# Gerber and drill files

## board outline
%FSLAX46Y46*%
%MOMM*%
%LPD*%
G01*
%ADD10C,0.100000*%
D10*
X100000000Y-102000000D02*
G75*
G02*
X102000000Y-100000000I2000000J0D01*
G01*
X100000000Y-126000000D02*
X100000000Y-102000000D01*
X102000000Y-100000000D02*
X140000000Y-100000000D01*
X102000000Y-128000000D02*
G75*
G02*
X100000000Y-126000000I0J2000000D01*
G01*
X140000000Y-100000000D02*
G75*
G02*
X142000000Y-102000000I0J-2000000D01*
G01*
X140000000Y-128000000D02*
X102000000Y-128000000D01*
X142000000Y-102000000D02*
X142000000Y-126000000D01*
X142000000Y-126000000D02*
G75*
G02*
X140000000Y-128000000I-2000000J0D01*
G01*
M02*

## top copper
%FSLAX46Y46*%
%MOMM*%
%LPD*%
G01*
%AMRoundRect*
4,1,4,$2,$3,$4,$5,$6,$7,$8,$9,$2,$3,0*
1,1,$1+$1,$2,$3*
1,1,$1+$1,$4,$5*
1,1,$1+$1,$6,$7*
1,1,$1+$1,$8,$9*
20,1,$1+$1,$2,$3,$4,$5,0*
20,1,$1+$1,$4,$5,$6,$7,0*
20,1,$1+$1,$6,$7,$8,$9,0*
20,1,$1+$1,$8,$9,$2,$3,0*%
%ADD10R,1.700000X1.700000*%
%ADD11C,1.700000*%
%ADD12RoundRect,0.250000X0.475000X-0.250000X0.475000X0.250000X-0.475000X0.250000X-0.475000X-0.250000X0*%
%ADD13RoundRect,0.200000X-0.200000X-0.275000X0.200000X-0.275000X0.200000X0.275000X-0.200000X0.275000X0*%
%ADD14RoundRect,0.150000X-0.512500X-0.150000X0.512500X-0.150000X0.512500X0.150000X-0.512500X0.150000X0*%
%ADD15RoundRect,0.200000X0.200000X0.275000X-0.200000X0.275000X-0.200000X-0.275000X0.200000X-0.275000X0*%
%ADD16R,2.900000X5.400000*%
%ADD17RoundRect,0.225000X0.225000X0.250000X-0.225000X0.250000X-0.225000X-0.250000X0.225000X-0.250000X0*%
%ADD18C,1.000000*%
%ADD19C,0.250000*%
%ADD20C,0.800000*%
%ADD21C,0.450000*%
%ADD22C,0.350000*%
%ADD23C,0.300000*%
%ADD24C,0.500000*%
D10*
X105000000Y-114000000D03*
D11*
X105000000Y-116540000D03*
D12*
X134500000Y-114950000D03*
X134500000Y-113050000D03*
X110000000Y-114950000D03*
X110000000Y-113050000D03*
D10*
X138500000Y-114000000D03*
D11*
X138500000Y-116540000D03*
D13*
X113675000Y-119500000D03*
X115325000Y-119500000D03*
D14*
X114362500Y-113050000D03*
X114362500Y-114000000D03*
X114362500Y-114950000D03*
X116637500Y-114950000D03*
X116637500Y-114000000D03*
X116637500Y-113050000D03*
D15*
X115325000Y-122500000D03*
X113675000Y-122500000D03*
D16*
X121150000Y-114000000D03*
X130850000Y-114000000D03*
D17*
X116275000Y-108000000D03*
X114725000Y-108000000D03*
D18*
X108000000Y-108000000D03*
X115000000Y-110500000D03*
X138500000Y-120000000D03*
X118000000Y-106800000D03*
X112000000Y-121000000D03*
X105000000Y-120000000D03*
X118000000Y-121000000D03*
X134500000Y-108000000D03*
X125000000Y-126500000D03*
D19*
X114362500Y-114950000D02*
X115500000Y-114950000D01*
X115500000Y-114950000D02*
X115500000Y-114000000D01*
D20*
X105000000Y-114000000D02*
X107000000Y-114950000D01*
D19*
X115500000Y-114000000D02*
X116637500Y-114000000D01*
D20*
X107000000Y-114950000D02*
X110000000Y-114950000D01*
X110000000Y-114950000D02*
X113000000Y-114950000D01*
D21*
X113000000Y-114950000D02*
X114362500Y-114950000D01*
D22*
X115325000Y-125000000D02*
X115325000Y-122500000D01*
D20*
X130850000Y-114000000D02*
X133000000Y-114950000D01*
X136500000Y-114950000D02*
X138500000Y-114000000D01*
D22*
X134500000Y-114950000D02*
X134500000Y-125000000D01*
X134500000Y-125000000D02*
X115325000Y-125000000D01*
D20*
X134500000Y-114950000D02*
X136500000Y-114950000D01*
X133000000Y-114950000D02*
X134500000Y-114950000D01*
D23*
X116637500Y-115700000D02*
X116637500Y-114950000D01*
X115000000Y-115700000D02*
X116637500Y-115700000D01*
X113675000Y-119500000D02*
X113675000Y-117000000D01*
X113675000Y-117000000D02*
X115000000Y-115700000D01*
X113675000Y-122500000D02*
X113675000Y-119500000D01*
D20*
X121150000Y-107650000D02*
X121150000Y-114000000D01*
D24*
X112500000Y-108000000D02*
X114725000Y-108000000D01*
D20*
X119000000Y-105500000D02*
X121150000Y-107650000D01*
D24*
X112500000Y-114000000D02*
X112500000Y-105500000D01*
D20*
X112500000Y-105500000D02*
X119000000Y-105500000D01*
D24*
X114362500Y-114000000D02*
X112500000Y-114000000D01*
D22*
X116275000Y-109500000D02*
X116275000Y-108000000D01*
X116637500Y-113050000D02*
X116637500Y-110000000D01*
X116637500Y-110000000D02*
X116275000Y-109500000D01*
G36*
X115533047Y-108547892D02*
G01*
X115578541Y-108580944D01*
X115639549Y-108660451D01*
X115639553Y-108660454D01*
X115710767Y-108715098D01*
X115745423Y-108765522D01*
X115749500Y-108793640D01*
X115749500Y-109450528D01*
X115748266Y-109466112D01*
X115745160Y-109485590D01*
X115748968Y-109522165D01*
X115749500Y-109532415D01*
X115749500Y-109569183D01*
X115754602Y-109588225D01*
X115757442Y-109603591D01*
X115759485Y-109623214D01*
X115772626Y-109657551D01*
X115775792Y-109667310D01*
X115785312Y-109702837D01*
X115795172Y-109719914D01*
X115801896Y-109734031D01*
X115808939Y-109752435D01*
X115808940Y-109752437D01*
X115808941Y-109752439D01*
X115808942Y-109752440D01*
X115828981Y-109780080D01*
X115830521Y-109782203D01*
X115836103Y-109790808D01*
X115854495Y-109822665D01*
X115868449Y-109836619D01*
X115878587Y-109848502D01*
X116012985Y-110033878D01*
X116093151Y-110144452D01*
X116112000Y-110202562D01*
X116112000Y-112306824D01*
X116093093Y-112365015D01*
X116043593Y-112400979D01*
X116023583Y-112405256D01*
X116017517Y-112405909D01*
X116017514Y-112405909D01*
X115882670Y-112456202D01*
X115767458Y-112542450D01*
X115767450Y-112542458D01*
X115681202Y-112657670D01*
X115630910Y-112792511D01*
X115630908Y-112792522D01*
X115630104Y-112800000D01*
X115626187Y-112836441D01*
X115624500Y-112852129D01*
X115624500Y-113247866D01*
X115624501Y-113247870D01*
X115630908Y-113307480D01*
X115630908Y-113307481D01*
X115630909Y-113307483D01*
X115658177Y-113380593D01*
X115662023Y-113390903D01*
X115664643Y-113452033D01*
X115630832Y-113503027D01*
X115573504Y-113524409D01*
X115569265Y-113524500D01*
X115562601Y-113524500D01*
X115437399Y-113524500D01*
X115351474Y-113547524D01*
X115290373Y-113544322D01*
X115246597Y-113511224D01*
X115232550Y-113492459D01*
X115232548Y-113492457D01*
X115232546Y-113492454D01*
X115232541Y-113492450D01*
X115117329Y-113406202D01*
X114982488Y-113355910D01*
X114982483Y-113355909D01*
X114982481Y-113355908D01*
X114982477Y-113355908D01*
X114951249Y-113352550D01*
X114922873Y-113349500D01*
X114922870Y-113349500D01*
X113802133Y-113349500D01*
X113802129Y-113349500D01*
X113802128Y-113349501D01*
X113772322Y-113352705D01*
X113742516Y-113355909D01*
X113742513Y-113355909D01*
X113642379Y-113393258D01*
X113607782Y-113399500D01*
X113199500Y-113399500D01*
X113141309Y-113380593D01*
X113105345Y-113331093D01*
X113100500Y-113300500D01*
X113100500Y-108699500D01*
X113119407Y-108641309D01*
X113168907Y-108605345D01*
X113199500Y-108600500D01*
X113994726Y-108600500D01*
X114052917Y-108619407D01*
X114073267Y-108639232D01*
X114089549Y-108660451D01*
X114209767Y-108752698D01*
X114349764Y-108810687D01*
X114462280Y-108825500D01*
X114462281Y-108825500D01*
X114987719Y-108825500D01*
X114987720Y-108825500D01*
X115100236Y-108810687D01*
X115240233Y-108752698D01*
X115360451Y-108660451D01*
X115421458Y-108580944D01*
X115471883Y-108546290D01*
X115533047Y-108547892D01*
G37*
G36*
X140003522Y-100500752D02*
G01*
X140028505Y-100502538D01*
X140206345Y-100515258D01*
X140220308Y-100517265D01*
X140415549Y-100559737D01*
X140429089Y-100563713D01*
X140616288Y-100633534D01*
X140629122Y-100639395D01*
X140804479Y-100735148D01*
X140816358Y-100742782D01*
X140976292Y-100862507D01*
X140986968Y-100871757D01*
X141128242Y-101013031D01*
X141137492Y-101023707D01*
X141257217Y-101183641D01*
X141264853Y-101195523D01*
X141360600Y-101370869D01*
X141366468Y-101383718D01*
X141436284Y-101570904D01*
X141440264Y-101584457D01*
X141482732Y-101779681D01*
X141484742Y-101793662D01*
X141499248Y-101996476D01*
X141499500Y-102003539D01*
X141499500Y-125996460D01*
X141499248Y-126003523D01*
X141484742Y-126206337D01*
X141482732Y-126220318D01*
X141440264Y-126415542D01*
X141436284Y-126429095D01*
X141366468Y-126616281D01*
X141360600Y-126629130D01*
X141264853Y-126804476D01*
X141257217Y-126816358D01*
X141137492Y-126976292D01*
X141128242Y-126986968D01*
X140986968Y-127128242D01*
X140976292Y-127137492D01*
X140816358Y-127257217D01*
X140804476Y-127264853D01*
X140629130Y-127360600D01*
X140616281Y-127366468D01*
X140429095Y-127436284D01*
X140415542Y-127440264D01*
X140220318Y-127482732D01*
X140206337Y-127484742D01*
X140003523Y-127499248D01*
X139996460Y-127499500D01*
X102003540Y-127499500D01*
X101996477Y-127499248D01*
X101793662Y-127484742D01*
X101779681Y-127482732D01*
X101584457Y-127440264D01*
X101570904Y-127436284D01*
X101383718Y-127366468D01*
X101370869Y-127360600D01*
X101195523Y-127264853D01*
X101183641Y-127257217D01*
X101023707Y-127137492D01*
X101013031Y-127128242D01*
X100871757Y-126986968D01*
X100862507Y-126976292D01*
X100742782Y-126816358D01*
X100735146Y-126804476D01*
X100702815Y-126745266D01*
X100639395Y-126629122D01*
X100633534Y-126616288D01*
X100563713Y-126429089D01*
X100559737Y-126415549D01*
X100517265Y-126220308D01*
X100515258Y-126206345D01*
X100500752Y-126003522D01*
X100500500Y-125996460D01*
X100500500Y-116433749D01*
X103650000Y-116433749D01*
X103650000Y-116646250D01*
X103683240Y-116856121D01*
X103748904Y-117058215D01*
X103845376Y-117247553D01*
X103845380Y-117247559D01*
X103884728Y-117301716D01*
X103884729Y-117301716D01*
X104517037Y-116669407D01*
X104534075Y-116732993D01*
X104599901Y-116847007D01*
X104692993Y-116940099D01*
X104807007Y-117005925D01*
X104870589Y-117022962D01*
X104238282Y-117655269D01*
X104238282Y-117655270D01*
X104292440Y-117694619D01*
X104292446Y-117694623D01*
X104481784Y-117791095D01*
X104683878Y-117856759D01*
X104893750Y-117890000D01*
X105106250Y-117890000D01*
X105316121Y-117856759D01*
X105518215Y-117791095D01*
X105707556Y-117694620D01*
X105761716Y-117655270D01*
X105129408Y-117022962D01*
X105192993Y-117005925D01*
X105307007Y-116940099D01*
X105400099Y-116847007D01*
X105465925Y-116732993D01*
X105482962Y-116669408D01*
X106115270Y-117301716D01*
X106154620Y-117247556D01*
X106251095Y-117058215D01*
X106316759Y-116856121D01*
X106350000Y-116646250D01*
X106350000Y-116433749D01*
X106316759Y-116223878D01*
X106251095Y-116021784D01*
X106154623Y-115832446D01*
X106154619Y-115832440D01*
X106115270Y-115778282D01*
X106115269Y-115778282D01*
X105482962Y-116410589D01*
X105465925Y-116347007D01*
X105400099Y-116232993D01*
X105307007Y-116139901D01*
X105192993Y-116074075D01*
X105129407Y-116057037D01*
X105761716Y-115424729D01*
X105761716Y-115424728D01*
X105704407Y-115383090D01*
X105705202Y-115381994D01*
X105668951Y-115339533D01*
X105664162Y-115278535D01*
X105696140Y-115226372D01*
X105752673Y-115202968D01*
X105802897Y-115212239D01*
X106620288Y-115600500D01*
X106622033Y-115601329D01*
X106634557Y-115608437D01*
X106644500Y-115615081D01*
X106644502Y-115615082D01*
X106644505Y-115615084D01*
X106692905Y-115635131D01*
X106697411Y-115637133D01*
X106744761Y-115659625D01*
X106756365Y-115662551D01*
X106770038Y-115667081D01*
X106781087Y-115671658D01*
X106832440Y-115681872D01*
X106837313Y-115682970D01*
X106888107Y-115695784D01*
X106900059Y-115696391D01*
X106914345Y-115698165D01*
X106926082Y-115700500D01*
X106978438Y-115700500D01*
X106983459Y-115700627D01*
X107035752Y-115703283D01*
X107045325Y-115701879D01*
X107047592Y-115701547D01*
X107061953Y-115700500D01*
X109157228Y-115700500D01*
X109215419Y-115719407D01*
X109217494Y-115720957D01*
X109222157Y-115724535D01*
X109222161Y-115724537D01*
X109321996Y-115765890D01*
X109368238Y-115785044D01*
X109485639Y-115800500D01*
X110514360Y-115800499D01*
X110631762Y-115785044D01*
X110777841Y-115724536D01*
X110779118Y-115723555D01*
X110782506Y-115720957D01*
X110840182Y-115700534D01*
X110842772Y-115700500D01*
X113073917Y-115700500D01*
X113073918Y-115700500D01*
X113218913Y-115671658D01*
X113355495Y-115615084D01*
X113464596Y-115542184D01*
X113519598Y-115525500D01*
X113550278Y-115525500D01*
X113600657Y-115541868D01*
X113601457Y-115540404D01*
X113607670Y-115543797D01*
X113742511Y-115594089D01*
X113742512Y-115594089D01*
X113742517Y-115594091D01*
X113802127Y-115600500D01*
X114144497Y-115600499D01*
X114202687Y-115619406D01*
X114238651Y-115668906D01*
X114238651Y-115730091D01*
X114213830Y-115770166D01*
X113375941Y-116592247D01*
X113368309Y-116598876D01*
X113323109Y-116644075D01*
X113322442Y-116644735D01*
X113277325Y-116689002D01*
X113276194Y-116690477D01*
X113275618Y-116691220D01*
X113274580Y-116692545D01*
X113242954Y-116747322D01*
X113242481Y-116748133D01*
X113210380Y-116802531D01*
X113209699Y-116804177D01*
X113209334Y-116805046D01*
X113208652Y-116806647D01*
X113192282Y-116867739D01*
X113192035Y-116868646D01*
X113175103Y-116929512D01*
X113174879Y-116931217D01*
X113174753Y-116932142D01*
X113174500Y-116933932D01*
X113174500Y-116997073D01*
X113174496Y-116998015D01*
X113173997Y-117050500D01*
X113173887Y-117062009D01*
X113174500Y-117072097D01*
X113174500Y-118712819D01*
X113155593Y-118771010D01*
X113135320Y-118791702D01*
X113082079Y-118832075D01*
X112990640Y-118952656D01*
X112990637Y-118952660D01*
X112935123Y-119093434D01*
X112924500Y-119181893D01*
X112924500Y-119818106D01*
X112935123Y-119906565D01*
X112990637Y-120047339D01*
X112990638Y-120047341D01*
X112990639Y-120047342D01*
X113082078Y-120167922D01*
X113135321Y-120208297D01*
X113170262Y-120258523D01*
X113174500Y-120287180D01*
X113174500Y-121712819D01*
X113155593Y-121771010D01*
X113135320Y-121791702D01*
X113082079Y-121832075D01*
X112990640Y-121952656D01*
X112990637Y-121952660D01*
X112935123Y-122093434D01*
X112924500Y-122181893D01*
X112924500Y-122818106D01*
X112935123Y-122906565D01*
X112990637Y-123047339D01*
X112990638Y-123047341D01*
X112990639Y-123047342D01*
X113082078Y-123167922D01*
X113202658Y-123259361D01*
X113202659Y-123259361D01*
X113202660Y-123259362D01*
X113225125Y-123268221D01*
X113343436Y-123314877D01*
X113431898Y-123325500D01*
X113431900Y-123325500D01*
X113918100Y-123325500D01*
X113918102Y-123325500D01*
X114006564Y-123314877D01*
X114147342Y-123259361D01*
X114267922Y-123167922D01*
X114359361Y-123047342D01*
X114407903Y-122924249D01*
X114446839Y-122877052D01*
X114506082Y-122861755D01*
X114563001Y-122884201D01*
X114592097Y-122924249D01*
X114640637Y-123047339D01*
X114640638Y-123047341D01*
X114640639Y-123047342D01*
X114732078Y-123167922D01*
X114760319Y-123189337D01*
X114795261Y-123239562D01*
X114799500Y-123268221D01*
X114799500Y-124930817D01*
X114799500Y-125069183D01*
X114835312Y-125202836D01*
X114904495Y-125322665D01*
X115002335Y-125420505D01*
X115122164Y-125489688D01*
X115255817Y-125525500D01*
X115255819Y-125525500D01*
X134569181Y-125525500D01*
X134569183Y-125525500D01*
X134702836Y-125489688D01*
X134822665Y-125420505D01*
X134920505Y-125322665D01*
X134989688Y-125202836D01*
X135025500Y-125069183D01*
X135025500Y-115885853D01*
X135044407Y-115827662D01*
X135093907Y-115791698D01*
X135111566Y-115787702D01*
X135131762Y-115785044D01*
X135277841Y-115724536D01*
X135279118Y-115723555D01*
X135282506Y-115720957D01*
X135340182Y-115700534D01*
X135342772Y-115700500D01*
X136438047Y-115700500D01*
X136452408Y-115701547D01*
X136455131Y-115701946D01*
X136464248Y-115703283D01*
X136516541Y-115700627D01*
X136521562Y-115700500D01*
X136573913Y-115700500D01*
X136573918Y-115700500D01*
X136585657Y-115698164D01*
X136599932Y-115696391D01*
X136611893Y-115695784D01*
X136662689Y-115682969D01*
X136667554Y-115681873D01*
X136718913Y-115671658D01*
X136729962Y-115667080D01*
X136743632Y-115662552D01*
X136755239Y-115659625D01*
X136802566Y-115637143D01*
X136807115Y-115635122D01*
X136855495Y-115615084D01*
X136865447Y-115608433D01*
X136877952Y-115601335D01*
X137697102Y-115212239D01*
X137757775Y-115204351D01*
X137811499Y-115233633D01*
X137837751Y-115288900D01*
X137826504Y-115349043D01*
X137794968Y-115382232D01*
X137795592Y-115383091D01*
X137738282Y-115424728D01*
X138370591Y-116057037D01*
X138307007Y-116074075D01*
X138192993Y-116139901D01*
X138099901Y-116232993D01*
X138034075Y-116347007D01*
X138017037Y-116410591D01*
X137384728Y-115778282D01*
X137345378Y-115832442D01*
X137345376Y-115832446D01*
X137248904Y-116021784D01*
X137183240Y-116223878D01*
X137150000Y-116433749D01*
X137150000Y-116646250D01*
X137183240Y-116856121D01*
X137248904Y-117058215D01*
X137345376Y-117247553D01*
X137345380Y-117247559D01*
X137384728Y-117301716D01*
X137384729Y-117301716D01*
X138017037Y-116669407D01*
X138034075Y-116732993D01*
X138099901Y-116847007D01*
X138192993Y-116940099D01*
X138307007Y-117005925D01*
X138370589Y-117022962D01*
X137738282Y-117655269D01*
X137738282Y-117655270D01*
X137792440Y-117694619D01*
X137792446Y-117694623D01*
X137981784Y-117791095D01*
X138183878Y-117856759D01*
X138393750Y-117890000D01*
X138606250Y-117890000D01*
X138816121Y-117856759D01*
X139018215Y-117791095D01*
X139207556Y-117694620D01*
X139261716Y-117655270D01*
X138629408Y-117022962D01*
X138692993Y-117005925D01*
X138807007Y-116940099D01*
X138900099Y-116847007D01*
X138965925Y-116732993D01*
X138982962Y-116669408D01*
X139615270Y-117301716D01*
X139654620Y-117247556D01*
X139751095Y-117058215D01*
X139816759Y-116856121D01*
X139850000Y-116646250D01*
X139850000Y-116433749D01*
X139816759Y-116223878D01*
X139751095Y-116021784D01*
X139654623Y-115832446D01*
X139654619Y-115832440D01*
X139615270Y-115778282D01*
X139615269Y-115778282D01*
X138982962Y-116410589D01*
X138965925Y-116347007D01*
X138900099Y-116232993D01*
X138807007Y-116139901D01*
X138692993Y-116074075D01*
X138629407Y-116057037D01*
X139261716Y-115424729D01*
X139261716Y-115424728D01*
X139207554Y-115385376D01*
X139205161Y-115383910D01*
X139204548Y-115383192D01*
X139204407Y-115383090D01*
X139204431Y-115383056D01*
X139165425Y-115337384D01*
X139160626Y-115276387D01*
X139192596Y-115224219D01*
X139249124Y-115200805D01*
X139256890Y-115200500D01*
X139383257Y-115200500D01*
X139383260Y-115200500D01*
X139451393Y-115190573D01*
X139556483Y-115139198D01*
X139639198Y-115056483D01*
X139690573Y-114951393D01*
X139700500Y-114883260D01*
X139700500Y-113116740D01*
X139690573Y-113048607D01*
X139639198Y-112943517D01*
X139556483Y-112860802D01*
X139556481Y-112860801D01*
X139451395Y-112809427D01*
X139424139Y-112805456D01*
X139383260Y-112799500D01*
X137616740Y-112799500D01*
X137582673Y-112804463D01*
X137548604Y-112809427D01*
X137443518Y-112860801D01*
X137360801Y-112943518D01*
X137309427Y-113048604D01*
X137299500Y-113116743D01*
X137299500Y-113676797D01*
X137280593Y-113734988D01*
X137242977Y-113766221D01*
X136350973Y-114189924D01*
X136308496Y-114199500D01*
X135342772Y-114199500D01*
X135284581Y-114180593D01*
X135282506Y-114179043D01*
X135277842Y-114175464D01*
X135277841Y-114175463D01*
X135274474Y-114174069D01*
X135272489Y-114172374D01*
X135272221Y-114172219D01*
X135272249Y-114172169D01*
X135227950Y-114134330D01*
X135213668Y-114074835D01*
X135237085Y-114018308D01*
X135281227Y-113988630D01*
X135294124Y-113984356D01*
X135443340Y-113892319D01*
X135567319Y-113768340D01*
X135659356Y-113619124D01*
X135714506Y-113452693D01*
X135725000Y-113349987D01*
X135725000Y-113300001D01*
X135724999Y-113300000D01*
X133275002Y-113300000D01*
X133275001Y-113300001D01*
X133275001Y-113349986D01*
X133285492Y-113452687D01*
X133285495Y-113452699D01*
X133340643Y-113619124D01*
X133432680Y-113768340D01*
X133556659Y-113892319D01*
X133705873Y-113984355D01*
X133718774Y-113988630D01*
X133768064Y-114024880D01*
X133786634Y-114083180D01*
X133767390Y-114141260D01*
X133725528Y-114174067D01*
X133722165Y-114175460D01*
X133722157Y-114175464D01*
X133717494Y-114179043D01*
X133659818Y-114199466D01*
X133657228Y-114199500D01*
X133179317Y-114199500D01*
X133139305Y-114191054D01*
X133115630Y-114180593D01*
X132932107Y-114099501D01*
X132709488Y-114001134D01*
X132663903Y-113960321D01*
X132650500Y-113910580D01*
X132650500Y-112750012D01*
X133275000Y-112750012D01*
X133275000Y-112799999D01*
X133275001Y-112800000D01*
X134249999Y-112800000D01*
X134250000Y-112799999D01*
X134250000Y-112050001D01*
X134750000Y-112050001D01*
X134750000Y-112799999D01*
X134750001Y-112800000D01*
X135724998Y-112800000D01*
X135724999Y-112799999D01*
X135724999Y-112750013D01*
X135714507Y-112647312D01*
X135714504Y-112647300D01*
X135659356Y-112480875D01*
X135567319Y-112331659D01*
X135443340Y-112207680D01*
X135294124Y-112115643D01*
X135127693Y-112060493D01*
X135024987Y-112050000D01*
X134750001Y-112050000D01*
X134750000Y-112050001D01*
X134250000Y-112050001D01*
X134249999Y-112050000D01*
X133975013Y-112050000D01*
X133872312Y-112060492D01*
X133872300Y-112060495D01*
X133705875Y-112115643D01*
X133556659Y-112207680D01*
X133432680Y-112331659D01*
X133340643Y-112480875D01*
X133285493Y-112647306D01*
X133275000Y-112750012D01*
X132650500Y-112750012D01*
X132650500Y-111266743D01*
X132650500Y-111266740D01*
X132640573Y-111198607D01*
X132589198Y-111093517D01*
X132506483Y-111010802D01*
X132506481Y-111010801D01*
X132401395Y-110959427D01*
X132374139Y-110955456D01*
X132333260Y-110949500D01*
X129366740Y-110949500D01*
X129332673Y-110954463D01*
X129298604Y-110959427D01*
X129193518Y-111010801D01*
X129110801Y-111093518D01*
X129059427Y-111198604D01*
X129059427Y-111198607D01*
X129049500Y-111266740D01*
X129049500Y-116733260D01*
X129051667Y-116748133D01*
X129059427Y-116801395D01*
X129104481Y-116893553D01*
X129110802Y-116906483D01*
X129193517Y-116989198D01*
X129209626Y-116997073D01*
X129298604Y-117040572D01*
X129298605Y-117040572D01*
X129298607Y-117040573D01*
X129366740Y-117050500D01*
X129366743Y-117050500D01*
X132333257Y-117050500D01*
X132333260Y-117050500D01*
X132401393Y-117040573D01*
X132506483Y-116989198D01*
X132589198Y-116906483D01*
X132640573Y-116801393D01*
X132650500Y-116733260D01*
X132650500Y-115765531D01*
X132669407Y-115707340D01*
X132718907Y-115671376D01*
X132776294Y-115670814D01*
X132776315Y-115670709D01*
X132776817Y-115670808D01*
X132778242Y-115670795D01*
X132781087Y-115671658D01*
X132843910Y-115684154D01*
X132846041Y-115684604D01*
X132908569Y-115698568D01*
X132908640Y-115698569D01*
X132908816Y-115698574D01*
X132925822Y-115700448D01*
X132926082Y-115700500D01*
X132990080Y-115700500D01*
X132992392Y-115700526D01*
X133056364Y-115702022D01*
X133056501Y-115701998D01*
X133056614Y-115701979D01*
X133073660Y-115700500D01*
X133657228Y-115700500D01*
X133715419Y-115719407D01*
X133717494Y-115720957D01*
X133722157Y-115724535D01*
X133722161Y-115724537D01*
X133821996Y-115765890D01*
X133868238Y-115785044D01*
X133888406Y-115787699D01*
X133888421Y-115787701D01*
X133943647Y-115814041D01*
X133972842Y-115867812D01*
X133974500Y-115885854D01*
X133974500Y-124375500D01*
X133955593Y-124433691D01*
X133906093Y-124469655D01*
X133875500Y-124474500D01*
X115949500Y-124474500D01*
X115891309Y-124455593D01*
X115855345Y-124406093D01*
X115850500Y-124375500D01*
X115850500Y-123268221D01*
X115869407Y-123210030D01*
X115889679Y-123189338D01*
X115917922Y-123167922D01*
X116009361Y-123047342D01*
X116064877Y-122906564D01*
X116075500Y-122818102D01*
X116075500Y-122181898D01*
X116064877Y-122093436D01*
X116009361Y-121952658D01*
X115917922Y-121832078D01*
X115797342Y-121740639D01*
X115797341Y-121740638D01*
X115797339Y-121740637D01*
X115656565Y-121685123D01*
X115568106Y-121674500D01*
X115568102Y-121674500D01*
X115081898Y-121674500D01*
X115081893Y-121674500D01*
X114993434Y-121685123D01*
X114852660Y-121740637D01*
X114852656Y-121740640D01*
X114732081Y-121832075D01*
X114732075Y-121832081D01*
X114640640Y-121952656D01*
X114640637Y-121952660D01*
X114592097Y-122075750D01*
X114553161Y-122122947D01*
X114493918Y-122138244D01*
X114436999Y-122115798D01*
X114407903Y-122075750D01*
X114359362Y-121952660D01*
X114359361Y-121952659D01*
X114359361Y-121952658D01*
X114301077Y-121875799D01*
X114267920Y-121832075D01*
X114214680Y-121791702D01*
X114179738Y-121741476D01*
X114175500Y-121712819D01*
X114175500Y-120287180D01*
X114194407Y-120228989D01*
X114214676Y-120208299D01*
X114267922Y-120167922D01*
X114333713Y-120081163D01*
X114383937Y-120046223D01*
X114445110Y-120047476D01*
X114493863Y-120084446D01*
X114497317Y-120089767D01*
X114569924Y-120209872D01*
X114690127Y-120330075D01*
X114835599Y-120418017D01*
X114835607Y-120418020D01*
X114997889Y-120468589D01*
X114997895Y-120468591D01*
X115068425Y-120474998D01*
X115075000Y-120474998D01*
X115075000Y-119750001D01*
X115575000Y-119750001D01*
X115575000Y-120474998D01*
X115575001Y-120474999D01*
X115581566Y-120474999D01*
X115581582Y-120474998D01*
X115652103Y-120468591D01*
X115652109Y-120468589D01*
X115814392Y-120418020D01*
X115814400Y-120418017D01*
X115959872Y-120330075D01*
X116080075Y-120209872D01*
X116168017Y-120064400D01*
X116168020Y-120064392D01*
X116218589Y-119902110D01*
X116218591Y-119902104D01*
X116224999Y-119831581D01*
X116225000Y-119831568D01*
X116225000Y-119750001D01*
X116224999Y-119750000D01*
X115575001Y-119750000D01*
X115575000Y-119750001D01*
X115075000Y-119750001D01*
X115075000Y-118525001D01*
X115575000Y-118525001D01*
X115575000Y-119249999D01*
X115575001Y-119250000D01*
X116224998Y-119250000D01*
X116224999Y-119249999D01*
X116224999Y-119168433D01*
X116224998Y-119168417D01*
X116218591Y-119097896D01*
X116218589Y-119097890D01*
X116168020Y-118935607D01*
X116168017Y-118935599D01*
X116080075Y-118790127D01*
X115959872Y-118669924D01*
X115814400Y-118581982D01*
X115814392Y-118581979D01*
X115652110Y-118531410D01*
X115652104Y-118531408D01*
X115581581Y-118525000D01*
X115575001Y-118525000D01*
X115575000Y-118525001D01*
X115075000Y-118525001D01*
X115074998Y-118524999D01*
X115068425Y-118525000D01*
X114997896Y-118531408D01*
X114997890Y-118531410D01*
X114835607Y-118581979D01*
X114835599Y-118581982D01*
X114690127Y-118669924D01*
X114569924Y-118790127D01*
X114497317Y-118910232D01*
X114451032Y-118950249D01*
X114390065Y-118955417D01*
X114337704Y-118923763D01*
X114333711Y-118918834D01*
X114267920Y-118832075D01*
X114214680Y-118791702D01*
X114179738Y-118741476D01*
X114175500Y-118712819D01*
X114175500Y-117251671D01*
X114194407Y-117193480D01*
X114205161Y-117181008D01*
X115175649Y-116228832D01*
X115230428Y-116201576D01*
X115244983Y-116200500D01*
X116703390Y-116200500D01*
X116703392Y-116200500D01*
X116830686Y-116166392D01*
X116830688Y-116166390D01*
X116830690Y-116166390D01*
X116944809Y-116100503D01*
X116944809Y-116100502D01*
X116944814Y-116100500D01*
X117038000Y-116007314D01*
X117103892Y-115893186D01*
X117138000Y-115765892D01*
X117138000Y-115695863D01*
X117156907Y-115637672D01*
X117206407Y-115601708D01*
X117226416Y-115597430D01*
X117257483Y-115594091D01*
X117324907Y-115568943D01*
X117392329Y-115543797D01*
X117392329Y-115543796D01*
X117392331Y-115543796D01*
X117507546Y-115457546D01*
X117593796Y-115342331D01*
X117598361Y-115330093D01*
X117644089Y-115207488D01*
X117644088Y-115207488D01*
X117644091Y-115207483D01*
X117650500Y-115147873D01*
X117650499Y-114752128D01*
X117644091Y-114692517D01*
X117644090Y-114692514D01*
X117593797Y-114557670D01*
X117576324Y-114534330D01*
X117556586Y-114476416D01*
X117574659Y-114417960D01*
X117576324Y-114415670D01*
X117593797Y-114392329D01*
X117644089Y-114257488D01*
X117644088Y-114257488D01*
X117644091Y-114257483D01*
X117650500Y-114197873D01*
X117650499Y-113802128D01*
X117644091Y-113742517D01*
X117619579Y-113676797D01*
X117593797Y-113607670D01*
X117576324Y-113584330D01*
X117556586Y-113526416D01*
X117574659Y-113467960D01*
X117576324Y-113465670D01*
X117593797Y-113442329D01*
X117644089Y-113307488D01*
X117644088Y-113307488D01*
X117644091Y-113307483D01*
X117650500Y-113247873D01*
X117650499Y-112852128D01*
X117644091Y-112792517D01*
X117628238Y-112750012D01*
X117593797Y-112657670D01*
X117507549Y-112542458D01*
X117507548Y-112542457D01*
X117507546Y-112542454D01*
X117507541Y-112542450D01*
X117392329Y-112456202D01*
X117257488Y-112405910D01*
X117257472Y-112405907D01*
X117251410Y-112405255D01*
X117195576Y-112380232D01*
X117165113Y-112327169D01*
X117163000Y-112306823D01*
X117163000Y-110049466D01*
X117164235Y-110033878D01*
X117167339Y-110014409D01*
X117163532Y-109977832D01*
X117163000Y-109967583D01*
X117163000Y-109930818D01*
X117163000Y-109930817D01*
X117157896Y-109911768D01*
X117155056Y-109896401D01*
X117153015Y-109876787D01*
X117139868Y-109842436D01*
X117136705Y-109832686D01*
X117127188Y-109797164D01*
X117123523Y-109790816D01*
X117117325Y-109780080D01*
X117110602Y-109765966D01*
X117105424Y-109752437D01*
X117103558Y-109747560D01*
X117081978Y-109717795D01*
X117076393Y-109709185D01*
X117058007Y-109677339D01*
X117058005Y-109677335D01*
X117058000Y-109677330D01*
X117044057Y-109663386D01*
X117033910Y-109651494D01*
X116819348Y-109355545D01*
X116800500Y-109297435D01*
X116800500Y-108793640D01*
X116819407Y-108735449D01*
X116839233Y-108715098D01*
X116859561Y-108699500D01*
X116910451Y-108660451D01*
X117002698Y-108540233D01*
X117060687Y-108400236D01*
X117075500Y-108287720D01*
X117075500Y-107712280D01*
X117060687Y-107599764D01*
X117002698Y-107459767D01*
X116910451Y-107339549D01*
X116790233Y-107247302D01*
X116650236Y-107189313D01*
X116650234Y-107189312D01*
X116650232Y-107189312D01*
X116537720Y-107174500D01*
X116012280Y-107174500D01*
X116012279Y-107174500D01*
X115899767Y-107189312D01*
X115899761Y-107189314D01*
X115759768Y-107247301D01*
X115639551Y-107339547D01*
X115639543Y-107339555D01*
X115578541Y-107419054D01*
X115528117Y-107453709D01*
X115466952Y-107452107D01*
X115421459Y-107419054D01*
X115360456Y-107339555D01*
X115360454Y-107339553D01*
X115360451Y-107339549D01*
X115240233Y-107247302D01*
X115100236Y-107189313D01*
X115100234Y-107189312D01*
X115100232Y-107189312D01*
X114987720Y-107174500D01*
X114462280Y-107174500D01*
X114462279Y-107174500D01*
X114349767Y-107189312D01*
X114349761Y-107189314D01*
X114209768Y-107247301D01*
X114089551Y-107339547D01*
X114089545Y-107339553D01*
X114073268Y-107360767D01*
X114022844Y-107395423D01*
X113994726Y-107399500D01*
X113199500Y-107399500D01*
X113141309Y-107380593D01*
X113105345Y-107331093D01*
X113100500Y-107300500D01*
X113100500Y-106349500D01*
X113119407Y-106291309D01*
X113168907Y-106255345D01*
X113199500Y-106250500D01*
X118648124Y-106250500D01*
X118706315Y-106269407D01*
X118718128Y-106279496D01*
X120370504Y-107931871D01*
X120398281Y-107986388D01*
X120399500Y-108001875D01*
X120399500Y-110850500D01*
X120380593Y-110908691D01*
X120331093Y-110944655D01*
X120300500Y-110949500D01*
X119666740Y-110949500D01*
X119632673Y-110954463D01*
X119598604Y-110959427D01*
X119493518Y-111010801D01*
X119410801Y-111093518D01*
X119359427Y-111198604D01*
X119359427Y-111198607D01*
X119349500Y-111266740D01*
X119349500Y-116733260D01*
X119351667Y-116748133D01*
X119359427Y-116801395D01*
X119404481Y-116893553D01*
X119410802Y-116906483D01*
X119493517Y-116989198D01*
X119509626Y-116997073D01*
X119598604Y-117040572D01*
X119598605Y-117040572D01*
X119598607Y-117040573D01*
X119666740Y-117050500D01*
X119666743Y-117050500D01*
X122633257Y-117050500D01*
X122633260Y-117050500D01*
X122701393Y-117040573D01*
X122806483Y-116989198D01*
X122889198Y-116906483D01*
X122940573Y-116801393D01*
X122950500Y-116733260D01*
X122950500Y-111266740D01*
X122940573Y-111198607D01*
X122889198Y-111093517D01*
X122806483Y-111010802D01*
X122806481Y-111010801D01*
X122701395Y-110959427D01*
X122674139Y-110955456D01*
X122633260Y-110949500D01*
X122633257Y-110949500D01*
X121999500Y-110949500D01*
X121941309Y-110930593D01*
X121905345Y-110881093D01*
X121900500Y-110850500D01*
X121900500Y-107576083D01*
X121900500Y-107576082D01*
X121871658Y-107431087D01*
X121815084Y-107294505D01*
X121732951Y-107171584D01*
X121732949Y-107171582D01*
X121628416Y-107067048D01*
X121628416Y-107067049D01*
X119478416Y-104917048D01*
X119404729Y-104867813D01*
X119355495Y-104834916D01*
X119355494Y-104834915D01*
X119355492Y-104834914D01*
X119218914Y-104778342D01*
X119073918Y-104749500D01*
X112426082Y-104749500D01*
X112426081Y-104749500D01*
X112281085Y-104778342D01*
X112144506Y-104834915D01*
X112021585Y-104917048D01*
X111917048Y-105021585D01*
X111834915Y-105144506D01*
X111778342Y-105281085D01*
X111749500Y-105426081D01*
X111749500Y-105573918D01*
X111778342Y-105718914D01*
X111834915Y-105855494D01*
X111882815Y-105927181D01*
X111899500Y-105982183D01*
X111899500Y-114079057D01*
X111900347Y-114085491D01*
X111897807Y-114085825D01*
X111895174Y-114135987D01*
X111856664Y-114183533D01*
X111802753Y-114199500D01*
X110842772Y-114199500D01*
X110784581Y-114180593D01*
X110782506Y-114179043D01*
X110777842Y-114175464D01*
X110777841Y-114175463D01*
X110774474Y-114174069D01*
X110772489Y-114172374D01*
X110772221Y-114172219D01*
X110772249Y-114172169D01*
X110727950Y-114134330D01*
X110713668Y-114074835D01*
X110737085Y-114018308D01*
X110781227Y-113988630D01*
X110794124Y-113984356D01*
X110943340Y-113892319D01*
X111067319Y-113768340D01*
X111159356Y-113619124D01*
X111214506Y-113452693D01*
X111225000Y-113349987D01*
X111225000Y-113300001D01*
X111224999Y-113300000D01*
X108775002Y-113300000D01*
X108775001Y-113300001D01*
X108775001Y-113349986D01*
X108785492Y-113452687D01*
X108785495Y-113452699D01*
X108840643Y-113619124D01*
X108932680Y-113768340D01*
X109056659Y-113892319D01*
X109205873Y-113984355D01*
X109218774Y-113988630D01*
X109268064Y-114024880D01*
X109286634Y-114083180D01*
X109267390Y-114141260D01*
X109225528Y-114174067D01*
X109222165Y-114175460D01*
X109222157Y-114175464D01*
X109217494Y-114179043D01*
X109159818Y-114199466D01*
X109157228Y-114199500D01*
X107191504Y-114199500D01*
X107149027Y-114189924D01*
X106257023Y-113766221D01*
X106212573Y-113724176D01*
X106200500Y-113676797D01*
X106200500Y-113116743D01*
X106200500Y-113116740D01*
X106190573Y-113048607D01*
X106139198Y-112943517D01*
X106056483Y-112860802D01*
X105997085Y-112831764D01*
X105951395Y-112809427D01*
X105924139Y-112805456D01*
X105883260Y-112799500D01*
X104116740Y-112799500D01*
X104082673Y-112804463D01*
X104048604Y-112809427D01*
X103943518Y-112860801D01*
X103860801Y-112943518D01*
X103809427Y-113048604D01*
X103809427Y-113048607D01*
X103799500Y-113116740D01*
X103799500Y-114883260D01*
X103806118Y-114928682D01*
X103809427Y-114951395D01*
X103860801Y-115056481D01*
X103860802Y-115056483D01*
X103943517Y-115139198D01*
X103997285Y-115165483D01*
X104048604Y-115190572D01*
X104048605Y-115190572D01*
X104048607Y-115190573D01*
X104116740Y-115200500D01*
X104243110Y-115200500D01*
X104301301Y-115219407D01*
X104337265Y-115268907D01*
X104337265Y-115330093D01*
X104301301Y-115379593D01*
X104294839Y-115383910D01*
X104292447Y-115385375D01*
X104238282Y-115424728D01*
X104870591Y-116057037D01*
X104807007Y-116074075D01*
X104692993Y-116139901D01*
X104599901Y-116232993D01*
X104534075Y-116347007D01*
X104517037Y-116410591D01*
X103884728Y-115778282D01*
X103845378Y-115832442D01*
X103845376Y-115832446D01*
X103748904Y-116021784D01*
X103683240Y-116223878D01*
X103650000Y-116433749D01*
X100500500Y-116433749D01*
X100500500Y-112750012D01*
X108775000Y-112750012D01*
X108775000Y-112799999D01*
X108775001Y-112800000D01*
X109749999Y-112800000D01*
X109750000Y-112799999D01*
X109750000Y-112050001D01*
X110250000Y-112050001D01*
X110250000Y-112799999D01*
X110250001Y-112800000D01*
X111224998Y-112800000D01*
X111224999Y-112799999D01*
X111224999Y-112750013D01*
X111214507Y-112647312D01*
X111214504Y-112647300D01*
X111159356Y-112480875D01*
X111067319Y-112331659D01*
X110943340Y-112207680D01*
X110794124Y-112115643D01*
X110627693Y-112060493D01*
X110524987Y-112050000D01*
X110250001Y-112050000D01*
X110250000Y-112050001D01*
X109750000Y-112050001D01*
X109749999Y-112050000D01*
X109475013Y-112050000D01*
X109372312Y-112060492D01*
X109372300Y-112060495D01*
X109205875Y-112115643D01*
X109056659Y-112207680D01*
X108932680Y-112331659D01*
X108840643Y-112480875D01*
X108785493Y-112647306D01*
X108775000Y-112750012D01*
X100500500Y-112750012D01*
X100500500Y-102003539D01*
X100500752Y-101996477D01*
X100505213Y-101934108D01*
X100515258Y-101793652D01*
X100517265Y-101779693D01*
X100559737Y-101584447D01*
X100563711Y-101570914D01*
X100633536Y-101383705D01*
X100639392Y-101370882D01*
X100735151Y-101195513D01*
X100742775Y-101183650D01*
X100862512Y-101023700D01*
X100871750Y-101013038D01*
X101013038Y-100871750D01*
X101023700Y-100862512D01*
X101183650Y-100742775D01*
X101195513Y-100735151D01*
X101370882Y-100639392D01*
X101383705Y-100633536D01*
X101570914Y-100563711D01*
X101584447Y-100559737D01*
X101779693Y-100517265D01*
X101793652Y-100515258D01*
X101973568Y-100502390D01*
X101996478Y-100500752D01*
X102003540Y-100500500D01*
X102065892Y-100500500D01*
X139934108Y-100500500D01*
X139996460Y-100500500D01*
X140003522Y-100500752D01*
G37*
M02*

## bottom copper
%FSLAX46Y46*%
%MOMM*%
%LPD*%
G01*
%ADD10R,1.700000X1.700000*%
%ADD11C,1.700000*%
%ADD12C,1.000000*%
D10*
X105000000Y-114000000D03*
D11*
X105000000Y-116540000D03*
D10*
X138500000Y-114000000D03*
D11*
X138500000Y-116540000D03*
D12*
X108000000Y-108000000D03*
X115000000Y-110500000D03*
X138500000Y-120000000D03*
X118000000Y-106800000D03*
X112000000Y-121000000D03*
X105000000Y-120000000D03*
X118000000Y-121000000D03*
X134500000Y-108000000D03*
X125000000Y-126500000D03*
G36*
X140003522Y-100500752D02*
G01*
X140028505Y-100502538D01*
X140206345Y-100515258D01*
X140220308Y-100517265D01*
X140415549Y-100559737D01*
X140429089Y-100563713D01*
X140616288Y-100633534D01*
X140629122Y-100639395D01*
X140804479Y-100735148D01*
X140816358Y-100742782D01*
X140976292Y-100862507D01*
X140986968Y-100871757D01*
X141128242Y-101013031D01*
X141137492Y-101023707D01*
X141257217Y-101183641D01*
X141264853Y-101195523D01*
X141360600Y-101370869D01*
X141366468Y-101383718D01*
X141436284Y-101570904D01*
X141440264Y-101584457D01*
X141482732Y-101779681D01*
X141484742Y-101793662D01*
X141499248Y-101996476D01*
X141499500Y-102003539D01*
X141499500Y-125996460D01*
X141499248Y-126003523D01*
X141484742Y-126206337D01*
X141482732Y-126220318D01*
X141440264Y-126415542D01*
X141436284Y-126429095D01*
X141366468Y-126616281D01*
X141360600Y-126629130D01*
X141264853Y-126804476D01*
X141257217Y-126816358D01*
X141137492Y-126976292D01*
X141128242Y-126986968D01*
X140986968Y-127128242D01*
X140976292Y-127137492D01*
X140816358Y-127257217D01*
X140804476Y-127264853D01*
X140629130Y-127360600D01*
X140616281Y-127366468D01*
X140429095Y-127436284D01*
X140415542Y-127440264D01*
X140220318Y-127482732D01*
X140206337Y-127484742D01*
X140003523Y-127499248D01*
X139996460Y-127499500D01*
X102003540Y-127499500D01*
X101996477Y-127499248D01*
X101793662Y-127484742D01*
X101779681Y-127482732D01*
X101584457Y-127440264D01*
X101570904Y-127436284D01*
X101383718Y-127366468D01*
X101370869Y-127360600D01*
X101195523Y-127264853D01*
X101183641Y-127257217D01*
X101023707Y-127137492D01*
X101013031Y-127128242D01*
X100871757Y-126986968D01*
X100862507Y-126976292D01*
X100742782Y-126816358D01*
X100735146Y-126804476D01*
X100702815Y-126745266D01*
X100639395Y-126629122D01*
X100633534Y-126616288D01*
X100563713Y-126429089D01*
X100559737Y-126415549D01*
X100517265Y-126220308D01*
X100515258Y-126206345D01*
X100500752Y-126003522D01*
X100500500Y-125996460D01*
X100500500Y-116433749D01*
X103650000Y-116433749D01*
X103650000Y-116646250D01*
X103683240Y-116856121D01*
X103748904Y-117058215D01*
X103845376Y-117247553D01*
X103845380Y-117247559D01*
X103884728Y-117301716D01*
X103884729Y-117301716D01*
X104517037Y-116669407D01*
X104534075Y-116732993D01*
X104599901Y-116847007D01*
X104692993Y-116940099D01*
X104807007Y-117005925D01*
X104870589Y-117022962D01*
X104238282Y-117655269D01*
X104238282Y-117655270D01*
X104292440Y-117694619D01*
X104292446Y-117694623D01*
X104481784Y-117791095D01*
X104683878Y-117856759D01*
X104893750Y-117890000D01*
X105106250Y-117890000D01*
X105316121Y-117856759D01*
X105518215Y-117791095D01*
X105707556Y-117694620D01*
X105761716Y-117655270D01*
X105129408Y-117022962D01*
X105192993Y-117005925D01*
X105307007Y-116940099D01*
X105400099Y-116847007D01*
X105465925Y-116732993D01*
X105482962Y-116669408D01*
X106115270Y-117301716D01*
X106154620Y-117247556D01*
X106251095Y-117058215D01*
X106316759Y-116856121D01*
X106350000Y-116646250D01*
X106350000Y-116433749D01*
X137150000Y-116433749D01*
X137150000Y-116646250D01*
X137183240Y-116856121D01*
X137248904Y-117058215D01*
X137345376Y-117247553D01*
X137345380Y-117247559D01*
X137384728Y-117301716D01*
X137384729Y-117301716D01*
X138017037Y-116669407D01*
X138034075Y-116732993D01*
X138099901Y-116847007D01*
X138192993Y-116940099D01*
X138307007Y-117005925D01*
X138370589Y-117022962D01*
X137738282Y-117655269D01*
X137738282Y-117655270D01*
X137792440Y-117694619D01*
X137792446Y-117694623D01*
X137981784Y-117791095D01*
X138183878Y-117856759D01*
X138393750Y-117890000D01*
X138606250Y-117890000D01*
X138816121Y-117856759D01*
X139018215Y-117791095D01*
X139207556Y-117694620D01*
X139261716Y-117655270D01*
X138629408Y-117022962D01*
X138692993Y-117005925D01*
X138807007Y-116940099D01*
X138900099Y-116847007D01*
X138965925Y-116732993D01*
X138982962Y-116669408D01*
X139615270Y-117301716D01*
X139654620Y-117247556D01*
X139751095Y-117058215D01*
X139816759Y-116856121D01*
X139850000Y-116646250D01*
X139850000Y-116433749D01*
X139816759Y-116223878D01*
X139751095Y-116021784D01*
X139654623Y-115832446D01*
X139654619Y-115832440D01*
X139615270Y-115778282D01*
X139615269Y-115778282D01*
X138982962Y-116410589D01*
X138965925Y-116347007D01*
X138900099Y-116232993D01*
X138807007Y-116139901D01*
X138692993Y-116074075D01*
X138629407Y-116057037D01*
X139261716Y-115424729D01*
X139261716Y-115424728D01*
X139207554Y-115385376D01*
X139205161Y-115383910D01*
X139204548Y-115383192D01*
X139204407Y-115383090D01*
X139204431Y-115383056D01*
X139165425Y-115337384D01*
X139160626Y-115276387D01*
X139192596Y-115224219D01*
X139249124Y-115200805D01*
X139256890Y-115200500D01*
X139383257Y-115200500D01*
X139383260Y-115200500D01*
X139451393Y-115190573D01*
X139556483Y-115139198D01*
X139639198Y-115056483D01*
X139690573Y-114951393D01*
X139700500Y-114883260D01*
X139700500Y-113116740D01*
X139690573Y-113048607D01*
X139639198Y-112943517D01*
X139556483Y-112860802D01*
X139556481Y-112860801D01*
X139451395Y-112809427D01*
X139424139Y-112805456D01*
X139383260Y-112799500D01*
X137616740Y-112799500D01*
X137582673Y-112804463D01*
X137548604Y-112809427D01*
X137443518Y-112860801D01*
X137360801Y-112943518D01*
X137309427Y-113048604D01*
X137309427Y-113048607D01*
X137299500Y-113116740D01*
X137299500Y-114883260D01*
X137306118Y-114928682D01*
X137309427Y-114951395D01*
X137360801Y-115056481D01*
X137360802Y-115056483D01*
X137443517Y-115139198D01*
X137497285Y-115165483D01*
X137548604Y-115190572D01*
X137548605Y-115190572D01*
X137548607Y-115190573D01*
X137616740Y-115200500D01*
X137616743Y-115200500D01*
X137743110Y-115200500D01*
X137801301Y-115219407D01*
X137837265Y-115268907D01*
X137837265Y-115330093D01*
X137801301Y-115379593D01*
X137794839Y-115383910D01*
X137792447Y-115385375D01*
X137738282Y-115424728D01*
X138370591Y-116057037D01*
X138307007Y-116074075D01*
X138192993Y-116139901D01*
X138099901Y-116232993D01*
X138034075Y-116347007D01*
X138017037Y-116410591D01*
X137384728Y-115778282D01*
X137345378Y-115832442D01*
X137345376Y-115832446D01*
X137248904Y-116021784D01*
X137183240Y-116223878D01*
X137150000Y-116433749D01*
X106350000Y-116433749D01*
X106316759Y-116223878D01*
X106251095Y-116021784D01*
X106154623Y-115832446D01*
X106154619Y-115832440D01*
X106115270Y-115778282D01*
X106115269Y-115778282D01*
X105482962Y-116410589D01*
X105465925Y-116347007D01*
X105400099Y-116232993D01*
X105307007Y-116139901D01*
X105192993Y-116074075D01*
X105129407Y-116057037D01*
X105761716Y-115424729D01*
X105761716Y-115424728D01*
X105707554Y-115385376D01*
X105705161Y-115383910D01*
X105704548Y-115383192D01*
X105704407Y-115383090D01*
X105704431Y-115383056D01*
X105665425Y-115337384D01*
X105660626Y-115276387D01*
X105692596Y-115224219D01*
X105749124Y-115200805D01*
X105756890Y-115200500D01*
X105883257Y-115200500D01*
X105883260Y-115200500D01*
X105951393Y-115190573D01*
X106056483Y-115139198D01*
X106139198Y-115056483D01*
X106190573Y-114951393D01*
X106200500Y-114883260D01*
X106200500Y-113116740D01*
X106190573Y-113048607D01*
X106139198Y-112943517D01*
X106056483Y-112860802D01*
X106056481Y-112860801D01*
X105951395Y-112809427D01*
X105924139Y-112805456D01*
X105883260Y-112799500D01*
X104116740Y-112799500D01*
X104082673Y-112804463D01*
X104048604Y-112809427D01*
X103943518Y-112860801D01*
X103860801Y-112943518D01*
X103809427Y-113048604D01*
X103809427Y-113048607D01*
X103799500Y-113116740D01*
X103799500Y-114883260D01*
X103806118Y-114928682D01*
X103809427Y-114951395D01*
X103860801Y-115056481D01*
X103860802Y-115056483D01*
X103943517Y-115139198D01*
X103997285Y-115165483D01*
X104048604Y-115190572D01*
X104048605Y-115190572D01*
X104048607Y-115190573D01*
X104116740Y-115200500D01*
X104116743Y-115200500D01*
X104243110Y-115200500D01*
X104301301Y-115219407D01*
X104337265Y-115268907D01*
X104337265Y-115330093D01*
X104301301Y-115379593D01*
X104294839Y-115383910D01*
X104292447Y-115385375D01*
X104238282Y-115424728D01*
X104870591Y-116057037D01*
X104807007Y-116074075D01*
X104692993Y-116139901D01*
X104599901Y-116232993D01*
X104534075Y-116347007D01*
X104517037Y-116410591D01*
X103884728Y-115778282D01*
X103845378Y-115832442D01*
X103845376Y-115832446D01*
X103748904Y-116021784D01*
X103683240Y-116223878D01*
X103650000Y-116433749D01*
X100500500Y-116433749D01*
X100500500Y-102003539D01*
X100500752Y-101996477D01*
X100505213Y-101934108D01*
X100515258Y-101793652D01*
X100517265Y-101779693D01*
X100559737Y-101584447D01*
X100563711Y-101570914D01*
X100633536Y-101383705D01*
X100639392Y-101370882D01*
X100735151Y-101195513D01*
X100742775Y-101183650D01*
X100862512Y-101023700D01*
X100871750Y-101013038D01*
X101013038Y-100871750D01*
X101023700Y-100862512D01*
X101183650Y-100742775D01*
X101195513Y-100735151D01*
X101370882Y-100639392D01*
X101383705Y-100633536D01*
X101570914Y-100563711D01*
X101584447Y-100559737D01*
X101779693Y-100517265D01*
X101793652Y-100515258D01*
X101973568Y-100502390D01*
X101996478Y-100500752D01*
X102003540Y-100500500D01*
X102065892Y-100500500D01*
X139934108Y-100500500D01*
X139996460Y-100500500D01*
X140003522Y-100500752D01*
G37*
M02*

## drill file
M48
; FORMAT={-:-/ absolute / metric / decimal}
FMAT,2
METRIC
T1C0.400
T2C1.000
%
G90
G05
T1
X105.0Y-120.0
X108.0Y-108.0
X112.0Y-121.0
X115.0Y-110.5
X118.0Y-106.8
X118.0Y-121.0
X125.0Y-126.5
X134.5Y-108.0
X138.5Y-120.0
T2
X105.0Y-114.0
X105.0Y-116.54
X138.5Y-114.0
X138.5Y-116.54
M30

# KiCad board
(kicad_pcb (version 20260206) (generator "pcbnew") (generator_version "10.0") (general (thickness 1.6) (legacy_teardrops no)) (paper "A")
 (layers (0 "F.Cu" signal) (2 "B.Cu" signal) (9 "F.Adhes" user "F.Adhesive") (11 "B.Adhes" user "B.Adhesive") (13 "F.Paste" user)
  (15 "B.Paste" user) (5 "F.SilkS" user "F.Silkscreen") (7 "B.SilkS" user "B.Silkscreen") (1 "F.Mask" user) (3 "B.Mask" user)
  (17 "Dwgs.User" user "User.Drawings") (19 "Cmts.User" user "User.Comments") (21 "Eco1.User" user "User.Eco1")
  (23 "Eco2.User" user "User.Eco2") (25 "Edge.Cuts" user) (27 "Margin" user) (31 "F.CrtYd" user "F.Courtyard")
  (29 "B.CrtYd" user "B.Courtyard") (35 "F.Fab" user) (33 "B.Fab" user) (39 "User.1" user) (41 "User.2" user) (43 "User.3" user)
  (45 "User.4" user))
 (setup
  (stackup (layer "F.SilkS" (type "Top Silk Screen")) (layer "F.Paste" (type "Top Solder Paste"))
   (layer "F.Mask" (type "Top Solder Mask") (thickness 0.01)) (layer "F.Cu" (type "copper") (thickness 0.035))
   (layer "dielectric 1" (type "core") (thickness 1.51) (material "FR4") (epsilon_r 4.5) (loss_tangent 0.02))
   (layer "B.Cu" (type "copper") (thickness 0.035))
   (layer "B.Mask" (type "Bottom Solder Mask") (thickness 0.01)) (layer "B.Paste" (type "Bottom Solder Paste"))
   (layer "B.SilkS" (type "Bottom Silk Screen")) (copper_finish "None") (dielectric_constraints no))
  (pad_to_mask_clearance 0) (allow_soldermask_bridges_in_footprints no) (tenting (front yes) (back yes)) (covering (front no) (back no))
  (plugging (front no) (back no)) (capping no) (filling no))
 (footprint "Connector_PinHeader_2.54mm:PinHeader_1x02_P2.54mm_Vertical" (layer "F.Cu") (at 105 114)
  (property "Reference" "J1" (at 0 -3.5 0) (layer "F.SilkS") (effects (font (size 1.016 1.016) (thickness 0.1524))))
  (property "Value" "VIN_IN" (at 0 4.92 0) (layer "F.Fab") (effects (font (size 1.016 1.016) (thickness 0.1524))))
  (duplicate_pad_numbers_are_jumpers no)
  (pad "1" thru_hole rect (at 0 0) (size 1.7 1.7) (drill 1) (layers "*.Cu" "*.Mask") (remove_unused_layers no) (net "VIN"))
  (pad "2" thru_hole circle (at 0 2.54) (size 1.7 1.7) (drill 1) (layers "*.Cu" "*.Mask") (remove_unused_layers no) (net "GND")))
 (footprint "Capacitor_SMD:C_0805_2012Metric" (layer "F.Cu") (at 134.5 114 90)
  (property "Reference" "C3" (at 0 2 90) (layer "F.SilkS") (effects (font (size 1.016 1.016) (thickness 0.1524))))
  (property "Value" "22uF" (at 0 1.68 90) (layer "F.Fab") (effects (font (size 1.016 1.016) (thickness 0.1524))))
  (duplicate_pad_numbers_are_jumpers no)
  (pad "1" smd roundrect (at -0.95 0 90) (size 1 1.45) (layers "F.Cu" "F.Mask" "F.Paste") (roundrect_rratio 0.25) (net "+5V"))
  (pad "2" smd roundrect (at 0.95 0 90) (size 1 1.45) (layers "F.Cu" "F.Mask" "F.Paste") (roundrect_rratio 0.25) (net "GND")))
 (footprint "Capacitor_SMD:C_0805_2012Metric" (layer "F.Cu") (at 110 114 90)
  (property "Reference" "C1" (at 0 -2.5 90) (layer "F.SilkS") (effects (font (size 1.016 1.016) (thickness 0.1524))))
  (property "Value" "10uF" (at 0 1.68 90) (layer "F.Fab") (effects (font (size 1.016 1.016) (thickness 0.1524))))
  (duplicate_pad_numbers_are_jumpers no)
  (pad "1" smd roundrect (at -0.95 0 90) (size 1 1.45) (layers "F.Cu" "F.Mask" "F.Paste") (roundrect_rratio 0.25) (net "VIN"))
  (pad "2" smd roundrect (at 0.95 0 90) (size 1 1.45) (layers "F.Cu" "F.Mask" "F.Paste") (roundrect_rratio 0.25) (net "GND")))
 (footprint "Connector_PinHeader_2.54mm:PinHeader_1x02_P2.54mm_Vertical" (layer "F.Cu") (at 138.5 114)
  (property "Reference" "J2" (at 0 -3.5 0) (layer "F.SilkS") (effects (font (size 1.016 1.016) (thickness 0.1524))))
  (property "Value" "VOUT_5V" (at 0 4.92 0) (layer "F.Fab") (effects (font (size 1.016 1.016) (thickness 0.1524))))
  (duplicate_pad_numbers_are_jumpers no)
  (pad "1" thru_hole rect (at 0 0) (size 1.7 1.7) (drill 1) (layers "*.Cu" "*.Mask") (remove_unused_layers no) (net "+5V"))
  (pad "2" thru_hole circle (at 0 2.54) (size 1.7 1.7) (drill 1) (layers "*.Cu" "*.Mask") (remove_unused_layers no) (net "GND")))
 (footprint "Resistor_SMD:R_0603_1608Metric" (layer "F.Cu") (at 114.5 119.5)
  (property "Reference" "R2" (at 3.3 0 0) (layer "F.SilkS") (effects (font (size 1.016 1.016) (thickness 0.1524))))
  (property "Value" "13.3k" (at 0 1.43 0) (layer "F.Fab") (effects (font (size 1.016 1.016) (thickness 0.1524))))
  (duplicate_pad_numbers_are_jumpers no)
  (pad "1" smd roundrect (at -0.825 0) (size 0.8 0.95) (layers "F.Cu" "F.Mask" "F.Paste") (roundrect_rratio 0.25) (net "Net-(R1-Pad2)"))
  (pad "2" smd roundrect (at 0.825 0) (size 0.8 0.95) (layers "F.Cu" "F.Mask" "F.Paste") (roundrect_rratio 0.25) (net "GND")))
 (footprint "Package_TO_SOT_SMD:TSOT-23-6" (layer "F.Cu") (at 115.5 114)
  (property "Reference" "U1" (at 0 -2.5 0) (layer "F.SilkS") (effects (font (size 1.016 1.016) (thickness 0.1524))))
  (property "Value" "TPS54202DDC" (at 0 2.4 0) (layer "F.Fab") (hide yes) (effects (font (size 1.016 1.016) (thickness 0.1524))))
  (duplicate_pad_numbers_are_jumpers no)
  (pad "1" smd roundrect (at -1.1375 -0.95) (size 1.325 0.6) (layers "F.Cu" "F.Mask" "F.Paste") (roundrect_rratio 0.25) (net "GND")
   (zone_connect 2))
  (pad "2" smd roundrect (at -1.1375 0) (size 1.325 0.6) (layers "F.Cu" "F.Mask" "F.Paste") (roundrect_rratio 0.25) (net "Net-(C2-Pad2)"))
  (pad "3" smd roundrect (at -1.1375 0.95) (size 1.325 0.6) (layers "F.Cu" "F.Mask" "F.Paste") (roundrect_rratio 0.25) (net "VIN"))
  (pad "4" smd roundrect (at 1.1375 0.95) (size 1.325 0.6) (layers "F.Cu" "F.Mask" "F.Paste") (roundrect_rratio 0.25) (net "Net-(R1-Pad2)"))
  (pad "5" smd roundrect (at 1.1375 0) (size 1.325 0.6) (layers "F.Cu" "F.Mask" "F.Paste") (roundrect_rratio 0.25) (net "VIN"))
  (pad "6" smd roundrect (at 1.1375 -0.95) (size 1.325 0.6) (layers "F.Cu" "F.Mask" "F.Paste") (roundrect_rratio 0.25) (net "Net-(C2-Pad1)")))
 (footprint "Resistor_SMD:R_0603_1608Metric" (layer "F.Cu") (at 114.5 122.5 180)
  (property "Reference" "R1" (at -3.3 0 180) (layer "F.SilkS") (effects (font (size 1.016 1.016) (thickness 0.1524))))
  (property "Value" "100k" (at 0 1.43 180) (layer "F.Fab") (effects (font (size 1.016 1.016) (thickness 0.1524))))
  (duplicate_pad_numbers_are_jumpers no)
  (pad "1" smd roundrect (at -0.825 0 180) (size 0.8 0.95) (layers "F.Cu" "F.Mask" "F.Paste") (roundrect_rratio 0.25) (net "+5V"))
  (pad "2" smd roundrect (at 0.825 0 180) (size 0.8 0.95) (layers "F.Cu" "F.Mask" "F.Paste") (roundrect_rratio 0.25) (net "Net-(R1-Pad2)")))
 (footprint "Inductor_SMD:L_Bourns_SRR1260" (layer "F.Cu") (at 126 114)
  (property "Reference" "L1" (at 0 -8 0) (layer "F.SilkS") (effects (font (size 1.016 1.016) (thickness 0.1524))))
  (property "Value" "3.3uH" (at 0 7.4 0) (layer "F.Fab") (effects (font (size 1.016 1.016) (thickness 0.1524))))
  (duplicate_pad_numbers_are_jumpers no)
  (pad "1" smd rect (at -4.85 0) (size 2.9 5.4) (layers "F.Cu" "F.Mask" "F.Paste") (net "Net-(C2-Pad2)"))
  (pad "2" smd rect (at 4.85 0) (size 2.9 5.4) (layers "F.Cu" "F.Mask" "F.Paste") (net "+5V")))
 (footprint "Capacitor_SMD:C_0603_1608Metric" (layer "F.Cu") (at 115.5 108 180)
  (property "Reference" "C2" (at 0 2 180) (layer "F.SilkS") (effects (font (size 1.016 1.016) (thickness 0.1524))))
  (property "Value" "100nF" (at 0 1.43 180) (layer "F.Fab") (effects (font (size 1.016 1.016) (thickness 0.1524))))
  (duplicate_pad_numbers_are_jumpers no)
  (pad "1" smd roundrect (at -0.775 0 180) (size 0.9 0.95) (layers "F.Cu" "F.Mask" "F.Paste") (roundrect_rratio 0.25) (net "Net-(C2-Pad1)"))
  (pad "2" smd roundrect (at 0.775 0 180) (size 0.9 0.95) (layers "F.Cu" "F.Mask" "F.Paste") (roundrect_rratio 0.25) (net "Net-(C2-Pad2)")))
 (gr_arc (start 100 102) (mid 100.585786 100.585786) (end 102 100) (stroke (width 0.1) (type default)) (layer "Edge.Cuts"))
 (gr_line (start 100 126) (end 100 102) (stroke (width 0.1) (type default)) (layer "Edge.Cuts"))
 (gr_line (start 102 100) (end 140 100) (stroke (width 0.1) (type default)) (layer "Edge.Cuts"))
 (gr_arc (start 102 128) (mid 100.585786 127.414214) (end 100 126) (stroke (width 0.1) (type default)) (layer "Edge.Cuts"))
 (gr_arc (start 140 100) (mid 141.414214 100.585786) (end 142 102) (stroke (width 0.1) (type default)) (layer "Edge.Cuts"))
 (gr_line (start 140 128) (end 102 128) (stroke (width 0.1) (type default)) (layer "Edge.Cuts"))
 (gr_line (start 142 102) (end 142 126) (stroke (width 0.1) (type default)) (layer "Edge.Cuts"))
 (gr_arc (start 142 126) (mid 141.414214 127.414214) (end 140 128) (stroke (width 0.1) (type default)) (layer "Edge.Cuts"))
 (segment (start 114.3625 114.95) (end 115.5 114.95) (width 0.25) (layer "F.Cu") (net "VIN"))
 (segment (start 115.5 114.95) (end 115.5 114) (width 0.25) (layer "F.Cu") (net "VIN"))
 (segment (start 105 114) (end 107 114.95) (width 0.8) (layer "F.Cu") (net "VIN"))
 (segment (start 115.5 114) (end 116.6375 114) (width 0.25) (layer "F.Cu") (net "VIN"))
 (segment (start 107 114.95) (end 110 114.95) (width 0.8) (layer "F.Cu") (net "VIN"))
 (segment (start 110 114.95) (end 113 114.95) (width 0.8) (layer "F.Cu") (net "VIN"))
 (segment (start 113 114.95) (end 114.3625 114.95) (width 0.45) (layer "F.Cu") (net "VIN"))
 (via (at 108 108) (size 1) (drill 0.4) (layers "F.Cu" "B.Cu") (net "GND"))
 (via (at 115 110.5) (size 1) (drill 0.4) (layers "F.Cu" "B.Cu") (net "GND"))
 (via (at 138.5 120) (size 1) (drill 0.4) (layers "F.Cu" "B.Cu") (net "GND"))
 (via (at 118 106.8) (size 1) (drill 0.4) (layers "F.Cu" "B.Cu") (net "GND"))
 (via (at 112 121) (size 1) (drill 0.4) (layers "F.Cu" "B.Cu") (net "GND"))
 (via (at 105 120) (size 1) (drill 0.4) (layers "F.Cu" "B.Cu") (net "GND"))
 (via (at 118 121) (size 1) (drill 0.4) (layers "F.Cu" "B.Cu") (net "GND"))
 (via (at 134.5 108) (size 1) (drill 0.4) (layers "F.Cu" "B.Cu") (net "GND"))
 (via (at 125 126.5) (size 1) (drill 0.4) (layers "F.Cu" "B.Cu") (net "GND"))
 (segment (start 115.325 125) (end 115.325 122.5) (width 0.35) (layer "F.Cu") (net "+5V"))
 (segment (start 130.85 114) (end 133 114.95) (width 0.8) (layer "F.Cu") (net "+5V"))
 (segment (start 136.5 114.95) (end 138.5 114) (width 0.8) (layer "F.Cu") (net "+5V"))
 (segment (start 134.5 114.95) (end 134.5 125) (width 0.35) (layer "F.Cu") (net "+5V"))
 (segment (start 134.5 125) (end 115.325 125) (width 0.35) (layer "F.Cu") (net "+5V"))
 (segment (start 134.5 114.95) (end 136.5 114.95) (width 0.8) (layer "F.Cu") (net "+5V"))
 (segment (start 133 114.95) (end 134.5 114.95) (width 0.8) (layer "F.Cu") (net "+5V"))
 (segment (start 116.6375 115.7) (end 116.6375 114.95) (width 0.3) (layer "F.Cu") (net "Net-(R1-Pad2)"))
 (segment (start 115 115.7) (end 116.6375 115.7) (width 0.3) (layer "F.Cu") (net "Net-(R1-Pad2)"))
 (segment (start 113.675 119.5) (end 113.675 117) (width 0.3) (layer "F.Cu") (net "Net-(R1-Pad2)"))
 (segment (start 113.675 117) (end 115 115.7) (width 0.3) (layer "F.Cu") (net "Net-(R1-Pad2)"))
 (segment (start 113.675 122.5) (end 113.675 119.5) (width 0.3) (layer "F.Cu") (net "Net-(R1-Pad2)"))
 (segment (start 121.15 107.65) (end 121.15 114) (width 0.8) (layer "F.Cu") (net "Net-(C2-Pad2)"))
 (segment (start 112.5 108) (end 114.725 108) (width 0.5) (layer "F.Cu") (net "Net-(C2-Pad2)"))
 (segment (start 119 105.5) (end 121.15 107.65) (width 0.8) (layer "F.Cu") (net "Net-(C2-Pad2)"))
 (segment (start 112.5 114) (end 112.5 105.5) (width 0.5) (layer "F.Cu") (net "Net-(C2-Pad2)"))
 (segment (start 112.5 105.5) (end 119 105.5) (width 0.8) (layer "F.Cu") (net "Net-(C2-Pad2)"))
 (segment (start 114.3625 114) (end 112.5 114) (width 0.5) (layer "F.Cu") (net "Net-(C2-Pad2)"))
 (segment (start 116.275 109.5) (end 116.275 108) (width 0.35) (layer "F.Cu") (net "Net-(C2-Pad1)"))
 (segment (start 116.6375 113.05) (end 116.6375 110) (width 0.35) (layer "F.Cu") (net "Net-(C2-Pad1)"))
 (segment (start 116.6375 110) (end 116.275 109.5) (width 0.35) (layer "F.Cu") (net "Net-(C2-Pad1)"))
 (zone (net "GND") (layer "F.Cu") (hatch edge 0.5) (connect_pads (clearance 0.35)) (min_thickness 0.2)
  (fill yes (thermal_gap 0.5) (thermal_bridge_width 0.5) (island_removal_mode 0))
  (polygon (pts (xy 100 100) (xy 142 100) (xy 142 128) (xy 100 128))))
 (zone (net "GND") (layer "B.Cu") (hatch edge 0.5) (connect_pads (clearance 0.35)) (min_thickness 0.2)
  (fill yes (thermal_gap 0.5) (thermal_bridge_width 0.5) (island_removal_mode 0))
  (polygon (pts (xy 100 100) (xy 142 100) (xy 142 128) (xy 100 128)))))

